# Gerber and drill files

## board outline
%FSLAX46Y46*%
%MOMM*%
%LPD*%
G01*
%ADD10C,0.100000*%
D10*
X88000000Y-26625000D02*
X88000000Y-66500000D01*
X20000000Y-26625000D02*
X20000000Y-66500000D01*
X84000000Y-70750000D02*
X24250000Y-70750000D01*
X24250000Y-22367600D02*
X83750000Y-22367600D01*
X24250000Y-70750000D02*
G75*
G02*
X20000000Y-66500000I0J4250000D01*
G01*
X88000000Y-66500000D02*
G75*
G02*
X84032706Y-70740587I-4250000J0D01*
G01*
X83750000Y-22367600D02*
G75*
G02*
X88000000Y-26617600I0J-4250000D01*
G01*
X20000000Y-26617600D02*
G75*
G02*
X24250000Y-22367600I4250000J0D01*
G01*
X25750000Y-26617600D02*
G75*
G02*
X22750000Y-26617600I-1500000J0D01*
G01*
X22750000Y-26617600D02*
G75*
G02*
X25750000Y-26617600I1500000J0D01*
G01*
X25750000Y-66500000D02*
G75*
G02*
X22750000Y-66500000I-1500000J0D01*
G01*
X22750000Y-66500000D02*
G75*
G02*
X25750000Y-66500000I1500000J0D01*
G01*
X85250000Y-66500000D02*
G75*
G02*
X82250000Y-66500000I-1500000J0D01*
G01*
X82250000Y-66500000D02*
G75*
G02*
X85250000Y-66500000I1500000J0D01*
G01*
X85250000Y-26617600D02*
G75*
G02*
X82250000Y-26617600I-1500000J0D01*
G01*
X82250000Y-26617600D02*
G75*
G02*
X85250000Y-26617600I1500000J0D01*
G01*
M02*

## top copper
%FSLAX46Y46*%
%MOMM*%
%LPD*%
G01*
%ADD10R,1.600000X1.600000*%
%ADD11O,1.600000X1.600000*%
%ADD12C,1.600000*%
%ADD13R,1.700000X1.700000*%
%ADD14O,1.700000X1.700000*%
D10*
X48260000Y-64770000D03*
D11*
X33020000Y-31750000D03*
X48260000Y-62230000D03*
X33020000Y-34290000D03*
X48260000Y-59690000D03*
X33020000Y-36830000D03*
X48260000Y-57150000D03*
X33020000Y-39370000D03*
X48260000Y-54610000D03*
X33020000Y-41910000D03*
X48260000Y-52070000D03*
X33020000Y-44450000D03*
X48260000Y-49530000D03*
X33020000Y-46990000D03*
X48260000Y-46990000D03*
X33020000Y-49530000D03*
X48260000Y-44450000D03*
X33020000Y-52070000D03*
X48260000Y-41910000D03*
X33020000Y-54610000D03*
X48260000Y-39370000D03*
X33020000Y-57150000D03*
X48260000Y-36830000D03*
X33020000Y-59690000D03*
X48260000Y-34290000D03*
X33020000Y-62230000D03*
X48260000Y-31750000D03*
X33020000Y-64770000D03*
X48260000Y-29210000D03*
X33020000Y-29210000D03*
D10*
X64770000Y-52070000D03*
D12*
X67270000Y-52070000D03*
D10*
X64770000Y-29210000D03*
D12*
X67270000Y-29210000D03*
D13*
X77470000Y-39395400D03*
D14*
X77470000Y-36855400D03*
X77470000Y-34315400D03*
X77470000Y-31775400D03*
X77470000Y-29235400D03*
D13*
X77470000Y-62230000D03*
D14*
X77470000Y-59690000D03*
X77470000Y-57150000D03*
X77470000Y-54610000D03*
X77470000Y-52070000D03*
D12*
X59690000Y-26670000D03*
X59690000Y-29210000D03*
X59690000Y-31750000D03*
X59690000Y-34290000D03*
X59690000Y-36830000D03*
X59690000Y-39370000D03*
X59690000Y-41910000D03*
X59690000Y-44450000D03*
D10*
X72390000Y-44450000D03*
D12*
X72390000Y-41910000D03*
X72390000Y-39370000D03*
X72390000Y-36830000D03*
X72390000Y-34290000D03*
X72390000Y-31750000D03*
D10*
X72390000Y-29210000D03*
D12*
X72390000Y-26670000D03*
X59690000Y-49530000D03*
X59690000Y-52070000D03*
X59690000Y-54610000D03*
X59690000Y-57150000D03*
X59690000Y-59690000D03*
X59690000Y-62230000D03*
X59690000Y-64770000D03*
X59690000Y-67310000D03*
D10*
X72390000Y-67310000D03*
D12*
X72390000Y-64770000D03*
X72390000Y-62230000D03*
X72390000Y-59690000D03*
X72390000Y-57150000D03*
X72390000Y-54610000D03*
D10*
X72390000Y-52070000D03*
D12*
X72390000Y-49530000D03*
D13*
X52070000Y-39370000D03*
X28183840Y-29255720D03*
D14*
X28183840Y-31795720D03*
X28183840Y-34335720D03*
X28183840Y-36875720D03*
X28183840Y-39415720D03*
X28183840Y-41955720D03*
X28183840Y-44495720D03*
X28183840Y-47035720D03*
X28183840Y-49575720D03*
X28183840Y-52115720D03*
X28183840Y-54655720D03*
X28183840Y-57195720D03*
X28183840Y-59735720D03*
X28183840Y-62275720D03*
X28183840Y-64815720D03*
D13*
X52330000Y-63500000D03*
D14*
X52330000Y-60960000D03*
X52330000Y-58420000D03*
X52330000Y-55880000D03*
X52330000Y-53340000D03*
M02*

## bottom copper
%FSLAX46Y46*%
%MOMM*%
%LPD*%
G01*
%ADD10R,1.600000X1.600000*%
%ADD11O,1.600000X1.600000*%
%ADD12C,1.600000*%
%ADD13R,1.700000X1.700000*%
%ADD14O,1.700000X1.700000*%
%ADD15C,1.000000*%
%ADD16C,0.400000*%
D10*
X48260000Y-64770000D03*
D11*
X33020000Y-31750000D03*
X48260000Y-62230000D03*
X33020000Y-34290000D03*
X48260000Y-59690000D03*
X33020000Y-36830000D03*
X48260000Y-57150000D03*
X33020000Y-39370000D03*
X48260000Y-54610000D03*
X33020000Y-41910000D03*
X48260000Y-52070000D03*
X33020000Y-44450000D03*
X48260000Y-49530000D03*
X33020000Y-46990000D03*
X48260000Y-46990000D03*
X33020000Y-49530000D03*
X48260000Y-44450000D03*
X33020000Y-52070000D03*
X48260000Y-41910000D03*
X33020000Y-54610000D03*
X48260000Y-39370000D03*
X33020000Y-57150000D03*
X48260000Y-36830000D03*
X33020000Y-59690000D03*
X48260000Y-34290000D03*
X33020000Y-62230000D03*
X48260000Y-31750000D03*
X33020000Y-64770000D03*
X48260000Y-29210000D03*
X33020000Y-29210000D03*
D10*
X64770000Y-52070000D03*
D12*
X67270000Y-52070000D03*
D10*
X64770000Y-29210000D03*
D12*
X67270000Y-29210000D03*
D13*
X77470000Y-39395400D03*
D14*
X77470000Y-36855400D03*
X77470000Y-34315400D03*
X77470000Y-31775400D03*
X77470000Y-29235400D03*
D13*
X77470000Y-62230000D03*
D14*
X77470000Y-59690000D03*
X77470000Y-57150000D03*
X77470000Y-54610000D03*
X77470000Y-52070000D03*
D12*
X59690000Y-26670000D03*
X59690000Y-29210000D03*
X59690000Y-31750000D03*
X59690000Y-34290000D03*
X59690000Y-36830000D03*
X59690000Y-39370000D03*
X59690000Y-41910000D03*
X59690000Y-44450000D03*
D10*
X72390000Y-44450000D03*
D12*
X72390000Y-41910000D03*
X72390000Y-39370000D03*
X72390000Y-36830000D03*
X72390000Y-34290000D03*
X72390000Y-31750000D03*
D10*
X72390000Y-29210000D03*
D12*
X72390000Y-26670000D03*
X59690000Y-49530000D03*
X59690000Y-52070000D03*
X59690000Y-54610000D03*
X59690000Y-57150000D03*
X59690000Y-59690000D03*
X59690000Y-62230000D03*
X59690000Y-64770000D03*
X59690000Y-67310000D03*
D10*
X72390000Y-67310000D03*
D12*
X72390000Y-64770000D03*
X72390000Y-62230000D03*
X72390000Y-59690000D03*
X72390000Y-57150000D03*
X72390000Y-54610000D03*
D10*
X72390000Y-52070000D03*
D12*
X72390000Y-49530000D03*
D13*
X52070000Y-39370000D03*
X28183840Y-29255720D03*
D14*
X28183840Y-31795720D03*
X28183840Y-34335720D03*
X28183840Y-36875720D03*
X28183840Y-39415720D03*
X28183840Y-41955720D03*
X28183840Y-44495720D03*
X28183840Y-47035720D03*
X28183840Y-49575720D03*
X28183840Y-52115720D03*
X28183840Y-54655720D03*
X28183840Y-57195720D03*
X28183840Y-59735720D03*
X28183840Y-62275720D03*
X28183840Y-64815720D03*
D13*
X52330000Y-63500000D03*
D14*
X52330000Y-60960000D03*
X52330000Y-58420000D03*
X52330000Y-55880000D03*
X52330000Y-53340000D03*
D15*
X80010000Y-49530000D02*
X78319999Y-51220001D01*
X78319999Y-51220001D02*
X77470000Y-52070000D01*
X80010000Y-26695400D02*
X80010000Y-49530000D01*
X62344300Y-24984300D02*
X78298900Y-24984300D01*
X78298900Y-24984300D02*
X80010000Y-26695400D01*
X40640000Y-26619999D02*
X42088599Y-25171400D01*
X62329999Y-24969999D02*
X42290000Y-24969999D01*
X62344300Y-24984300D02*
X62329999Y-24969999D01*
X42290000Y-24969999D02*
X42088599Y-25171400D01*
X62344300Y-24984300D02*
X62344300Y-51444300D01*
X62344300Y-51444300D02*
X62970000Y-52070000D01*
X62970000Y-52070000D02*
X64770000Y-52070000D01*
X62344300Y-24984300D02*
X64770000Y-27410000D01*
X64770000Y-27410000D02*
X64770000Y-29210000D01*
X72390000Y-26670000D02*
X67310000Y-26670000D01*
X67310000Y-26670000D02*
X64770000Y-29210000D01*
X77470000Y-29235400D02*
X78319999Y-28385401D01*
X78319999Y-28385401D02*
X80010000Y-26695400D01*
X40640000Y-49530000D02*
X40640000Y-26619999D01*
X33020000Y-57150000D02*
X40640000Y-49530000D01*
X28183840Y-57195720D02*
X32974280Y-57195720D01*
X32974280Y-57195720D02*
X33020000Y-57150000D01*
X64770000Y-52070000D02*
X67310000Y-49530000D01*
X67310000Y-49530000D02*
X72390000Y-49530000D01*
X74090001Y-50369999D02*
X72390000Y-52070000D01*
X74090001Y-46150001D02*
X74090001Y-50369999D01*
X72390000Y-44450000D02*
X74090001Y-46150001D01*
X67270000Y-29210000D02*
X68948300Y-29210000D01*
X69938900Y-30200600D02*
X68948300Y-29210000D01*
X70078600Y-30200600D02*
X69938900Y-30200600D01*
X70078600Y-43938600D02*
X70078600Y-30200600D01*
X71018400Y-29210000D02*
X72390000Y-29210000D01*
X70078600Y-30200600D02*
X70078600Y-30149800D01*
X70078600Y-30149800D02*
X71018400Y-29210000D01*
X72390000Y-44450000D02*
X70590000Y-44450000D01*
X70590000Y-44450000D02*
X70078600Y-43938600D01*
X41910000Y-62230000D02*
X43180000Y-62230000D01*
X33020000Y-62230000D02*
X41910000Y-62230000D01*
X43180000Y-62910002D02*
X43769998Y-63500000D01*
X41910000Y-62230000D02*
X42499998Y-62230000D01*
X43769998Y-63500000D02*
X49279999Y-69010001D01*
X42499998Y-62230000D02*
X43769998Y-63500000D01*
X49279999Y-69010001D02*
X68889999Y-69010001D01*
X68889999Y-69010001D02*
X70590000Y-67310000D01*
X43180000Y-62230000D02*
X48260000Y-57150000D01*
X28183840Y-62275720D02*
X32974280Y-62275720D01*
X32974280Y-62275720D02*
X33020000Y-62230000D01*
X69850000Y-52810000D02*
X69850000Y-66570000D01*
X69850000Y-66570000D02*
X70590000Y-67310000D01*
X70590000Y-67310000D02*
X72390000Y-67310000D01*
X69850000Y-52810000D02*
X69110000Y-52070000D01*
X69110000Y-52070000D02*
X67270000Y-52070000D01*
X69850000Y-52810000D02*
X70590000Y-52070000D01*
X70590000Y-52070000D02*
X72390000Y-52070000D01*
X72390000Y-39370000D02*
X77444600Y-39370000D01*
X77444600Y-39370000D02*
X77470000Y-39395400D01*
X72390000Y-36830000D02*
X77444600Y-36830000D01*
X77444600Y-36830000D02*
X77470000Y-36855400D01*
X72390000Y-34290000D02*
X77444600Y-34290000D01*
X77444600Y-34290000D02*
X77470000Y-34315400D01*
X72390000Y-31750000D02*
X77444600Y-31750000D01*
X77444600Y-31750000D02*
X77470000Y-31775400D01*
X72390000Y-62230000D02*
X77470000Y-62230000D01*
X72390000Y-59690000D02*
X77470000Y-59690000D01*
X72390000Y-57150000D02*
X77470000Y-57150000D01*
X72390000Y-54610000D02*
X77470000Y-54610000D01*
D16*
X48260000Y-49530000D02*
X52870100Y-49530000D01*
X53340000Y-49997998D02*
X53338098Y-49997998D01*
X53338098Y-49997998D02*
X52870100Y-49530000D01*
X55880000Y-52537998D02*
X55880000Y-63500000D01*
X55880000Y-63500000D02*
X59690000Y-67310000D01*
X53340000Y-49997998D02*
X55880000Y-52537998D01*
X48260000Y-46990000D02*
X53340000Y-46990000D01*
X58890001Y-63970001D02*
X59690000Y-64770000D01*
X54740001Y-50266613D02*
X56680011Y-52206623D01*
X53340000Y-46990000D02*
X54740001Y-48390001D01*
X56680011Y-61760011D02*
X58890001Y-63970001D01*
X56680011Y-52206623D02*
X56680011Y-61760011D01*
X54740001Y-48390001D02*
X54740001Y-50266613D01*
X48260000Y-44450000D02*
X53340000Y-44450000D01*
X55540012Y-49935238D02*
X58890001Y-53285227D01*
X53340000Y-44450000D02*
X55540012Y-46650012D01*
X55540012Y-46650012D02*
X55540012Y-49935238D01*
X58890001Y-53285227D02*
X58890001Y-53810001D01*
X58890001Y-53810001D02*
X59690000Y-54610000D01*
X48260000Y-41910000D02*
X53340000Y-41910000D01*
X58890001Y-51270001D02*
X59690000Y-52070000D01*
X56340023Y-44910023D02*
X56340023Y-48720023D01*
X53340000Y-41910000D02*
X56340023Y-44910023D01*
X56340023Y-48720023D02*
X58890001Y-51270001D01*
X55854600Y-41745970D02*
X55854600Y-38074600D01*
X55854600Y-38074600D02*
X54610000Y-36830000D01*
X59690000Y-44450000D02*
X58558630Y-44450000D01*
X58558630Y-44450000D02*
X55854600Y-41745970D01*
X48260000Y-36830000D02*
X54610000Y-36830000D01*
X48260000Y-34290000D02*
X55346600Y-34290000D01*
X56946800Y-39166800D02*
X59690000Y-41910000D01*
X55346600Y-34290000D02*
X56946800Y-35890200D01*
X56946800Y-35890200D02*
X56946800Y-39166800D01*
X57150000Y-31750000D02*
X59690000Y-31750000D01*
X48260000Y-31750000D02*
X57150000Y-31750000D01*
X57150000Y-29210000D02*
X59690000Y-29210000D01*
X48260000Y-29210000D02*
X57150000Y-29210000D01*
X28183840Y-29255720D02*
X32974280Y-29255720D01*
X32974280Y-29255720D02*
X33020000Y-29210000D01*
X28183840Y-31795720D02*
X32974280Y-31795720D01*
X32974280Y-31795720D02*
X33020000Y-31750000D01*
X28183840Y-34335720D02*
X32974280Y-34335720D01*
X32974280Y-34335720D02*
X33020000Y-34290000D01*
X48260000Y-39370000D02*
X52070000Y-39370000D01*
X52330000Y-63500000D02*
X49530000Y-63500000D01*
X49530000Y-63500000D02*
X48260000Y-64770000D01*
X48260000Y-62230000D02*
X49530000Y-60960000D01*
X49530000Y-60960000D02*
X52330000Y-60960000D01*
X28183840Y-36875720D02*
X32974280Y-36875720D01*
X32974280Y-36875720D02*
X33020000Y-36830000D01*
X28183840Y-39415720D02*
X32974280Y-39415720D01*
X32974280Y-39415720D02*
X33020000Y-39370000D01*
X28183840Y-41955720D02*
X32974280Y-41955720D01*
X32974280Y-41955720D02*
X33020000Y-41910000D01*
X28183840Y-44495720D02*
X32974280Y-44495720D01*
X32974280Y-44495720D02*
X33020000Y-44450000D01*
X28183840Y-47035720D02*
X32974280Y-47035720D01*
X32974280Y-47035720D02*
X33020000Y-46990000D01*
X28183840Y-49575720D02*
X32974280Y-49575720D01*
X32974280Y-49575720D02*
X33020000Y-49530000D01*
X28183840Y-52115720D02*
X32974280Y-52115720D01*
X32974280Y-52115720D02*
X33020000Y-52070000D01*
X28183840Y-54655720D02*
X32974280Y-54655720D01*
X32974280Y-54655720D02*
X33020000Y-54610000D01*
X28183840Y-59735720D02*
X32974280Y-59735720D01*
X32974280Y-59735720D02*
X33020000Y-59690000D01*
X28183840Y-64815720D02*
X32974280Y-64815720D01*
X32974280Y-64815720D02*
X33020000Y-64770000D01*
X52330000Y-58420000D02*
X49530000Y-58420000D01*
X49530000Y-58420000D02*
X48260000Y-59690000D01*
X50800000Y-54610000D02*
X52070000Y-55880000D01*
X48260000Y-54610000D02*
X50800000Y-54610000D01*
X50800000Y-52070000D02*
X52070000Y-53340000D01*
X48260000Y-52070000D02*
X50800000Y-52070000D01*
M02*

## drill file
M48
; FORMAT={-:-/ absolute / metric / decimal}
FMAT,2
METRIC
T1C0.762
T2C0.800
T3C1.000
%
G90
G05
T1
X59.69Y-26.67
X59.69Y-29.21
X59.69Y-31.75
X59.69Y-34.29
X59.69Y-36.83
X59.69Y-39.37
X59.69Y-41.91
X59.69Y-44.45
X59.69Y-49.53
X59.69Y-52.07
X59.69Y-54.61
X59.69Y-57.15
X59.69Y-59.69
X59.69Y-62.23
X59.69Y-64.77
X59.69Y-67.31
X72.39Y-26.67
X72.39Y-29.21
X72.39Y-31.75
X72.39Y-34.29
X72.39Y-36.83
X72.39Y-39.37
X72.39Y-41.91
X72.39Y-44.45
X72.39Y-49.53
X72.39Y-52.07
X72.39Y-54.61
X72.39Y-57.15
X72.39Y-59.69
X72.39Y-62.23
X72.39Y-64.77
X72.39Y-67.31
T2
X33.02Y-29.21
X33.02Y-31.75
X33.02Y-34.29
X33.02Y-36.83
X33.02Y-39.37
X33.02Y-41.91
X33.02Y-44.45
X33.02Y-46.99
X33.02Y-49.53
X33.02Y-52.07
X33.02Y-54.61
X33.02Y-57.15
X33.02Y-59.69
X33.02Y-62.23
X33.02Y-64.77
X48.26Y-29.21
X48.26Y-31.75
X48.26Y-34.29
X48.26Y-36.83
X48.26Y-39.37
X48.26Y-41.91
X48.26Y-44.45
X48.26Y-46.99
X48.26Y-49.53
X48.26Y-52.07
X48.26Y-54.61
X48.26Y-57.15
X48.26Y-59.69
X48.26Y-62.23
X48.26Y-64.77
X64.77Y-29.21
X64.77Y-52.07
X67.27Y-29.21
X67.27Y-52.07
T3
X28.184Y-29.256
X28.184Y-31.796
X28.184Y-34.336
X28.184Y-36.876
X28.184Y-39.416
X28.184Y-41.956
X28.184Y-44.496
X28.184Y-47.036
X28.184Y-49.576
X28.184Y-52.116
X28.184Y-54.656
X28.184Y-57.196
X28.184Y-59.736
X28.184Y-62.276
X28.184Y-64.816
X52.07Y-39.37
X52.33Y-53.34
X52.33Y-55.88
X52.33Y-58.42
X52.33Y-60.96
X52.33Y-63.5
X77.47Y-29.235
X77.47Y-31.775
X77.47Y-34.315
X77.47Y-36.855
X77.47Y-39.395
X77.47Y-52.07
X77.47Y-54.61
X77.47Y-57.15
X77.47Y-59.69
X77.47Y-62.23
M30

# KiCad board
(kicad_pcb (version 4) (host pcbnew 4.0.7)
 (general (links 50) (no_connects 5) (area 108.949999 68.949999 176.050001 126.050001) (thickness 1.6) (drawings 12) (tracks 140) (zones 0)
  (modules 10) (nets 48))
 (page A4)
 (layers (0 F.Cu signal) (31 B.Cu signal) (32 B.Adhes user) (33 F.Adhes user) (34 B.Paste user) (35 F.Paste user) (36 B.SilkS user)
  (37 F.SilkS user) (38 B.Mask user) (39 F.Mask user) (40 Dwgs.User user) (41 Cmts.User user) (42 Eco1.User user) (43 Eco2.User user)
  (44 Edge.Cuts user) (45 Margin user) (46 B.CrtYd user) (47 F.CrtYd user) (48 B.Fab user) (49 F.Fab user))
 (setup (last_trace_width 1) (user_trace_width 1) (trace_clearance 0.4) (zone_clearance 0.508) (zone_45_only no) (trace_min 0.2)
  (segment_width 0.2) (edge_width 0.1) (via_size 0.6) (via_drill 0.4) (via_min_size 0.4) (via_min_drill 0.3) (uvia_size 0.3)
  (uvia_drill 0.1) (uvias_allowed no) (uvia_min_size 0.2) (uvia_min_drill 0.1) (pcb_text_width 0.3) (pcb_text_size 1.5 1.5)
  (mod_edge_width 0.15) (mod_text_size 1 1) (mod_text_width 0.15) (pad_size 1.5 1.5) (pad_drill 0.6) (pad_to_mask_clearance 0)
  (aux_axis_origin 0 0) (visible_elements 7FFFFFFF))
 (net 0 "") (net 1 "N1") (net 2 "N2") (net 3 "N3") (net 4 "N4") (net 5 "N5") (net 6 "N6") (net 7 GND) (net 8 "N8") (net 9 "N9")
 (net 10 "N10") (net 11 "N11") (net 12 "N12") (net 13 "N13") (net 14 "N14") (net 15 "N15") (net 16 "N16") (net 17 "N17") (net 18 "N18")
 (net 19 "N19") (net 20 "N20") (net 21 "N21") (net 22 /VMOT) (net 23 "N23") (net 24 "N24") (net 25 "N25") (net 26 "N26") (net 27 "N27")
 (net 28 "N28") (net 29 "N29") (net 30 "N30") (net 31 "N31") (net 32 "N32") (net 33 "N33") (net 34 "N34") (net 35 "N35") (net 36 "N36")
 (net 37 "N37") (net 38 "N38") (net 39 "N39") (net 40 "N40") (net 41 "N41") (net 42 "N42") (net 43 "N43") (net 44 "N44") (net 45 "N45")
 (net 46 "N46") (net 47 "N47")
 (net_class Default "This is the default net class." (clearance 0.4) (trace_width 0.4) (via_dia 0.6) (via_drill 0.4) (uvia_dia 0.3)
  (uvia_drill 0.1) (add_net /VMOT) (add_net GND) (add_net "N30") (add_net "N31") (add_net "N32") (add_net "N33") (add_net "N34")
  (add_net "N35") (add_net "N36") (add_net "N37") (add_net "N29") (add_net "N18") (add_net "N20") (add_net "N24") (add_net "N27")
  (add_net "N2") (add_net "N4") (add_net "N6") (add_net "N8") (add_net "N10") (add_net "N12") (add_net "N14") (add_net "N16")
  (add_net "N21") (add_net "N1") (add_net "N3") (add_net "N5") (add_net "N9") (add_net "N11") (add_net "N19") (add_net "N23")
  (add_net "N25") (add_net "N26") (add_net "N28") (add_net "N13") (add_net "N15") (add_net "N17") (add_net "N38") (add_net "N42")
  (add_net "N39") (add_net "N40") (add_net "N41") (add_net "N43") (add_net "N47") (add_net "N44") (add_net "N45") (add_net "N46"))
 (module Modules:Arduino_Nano (layer F.Cu) (at 48.26 64.77 180)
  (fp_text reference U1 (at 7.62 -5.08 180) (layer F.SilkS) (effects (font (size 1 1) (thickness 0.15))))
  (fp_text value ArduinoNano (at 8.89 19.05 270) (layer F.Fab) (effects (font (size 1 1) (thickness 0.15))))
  (pad 1 thru_hole rect (at 0 0 180) (size 1.6 1.6) (drill 0.8) (layers *.Cu *.Mask) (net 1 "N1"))
  (pad 17 thru_hole oval (at 15.24 33.02 180) (size 1.6 1.6) (drill 0.8) (layers *.Cu *.Mask) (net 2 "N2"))
  (pad 2 thru_hole oval (at 0 2.54 180) (size 1.6 1.6) (drill 0.8) (layers *.Cu *.Mask) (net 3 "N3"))
  (pad 18 thru_hole oval (at 15.24 30.48 180) (size 1.6 1.6) (drill 0.8) (layers *.Cu *.Mask) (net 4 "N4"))
  (pad 3 thru_hole oval (at 0 5.08 180) (size 1.6 1.6) (drill 0.8) (layers *.Cu *.Mask) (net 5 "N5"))
  (pad 19 thru_hole oval (at 15.24 27.94 180) (size 1.6 1.6) (drill 0.8) (layers *.Cu *.Mask) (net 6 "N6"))
  (pad 4 thru_hole oval (at 0 7.62 180) (size 1.6 1.6) (drill 0.8) (layers *.Cu *.Mask) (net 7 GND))
  (pad 20 thru_hole oval (at 15.24 25.4 180) (size 1.6 1.6) (drill 0.8) (layers *.Cu *.Mask) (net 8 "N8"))
  (pad 5 thru_hole oval (at 0 10.16 180) (size 1.6 1.6) (drill 0.8) (layers *.Cu *.Mask) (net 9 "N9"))
  (pad 21 thru_hole oval (at 15.24 22.86 180) (size 1.6 1.6) (drill 0.8) (layers *.Cu *.Mask) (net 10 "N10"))
  (pad 6 thru_hole oval (at 0 12.7 180) (size 1.6 1.6) (drill 0.8) (layers *.Cu *.Mask) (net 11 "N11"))
  (pad 22 thru_hole oval (at 15.24 20.32 180) (size 1.6 1.6) (drill 0.8) (layers *.Cu *.Mask) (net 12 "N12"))
  (pad 7 thru_hole oval (at 0 15.24 180) (size 1.6 1.6) (drill 0.8) (layers *.Cu *.Mask) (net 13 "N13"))
  (pad 23 thru_hole oval (at 15.24 17.78 180) (size 1.6 1.6) (drill 0.8) (layers *.Cu *.Mask) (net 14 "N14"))
  (pad 8 thru_hole oval (at 0 17.78 180) (size 1.6 1.6) (drill 0.8) (layers *.Cu *.Mask) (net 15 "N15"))
  (pad 24 thru_hole oval (at 15.24 15.24 180) (size 1.6 1.6) (drill 0.8) (layers *.Cu *.Mask) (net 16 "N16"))
  (pad 9 thru_hole oval (at 0 20.32 180) (size 1.6 1.6) (drill 0.8) (layers *.Cu *.Mask) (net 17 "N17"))
  (pad 25 thru_hole oval (at 15.24 12.7 180) (size 1.6 1.6) (drill 0.8) (layers *.Cu *.Mask) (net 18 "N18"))
  (pad 10 thru_hole oval (at 0 22.86 180) (size 1.6 1.6) (drill 0.8) (layers *.Cu *.Mask) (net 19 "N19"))
  (pad 26 thru_hole oval (at 15.24 10.16 180) (size 1.6 1.6) (drill 0.8) (layers *.Cu *.Mask) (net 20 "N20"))
  (pad 11 thru_hole oval (at 0 25.4 180) (size 1.6 1.6) (drill 0.8) (layers *.Cu *.Mask) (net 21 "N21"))
  (pad 27 thru_hole oval (at 15.24 7.62 180) (size 1.6 1.6) (drill 0.8) (layers *.Cu *.Mask) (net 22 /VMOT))
  (pad 12 thru_hole oval (at 0 27.94 180) (size 1.6 1.6) (drill 0.8) (layers *.Cu *.Mask) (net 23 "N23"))
  (pad 28 thru_hole oval (at 15.24 5.08 180) (size 1.6 1.6) (drill 0.8) (layers *.Cu *.Mask) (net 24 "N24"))
  (pad 13 thru_hole oval (at 0 30.48 180) (size 1.6 1.6) (drill 0.8) (layers *.Cu *.Mask) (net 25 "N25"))
  (pad 29 thru_hole oval (at 15.24 2.54 180) (size 1.6 1.6) (drill 0.8) (layers *.Cu *.Mask) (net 7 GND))
  (pad 14 thru_hole oval (at 0 33.02 180) (size 1.6 1.6) (drill 0.8) (layers *.Cu *.Mask) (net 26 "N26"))
  (pad 30 thru_hole oval (at 15.24 0 180) (size 1.6 1.6) (drill 0.8) (layers *.Cu *.Mask) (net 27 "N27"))
  (pad 15 thru_hole oval (at 0 35.56 180) (size 1.6 1.6) (drill 0.8) (layers *.Cu *.Mask) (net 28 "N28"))
  (pad 16 thru_hole oval (at 15.24 35.56 180) (size 1.6 1.6) (drill 0.8) (layers *.Cu *.Mask) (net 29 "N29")))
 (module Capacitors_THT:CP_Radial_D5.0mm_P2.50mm (layer F.Cu) (at 64.77 52.07)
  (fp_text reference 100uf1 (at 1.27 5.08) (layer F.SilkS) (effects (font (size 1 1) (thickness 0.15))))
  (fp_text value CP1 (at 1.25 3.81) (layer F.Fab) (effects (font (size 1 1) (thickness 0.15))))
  (pad 1 thru_hole rect (at 0 0) (size 1.6 1.6) (drill 0.8) (layers *.Cu *.Mask) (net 22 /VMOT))
  (pad 2 thru_hole circle (at 2.5 0) (size 1.6 1.6) (drill 0.8) (layers *.Cu *.Mask) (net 7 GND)))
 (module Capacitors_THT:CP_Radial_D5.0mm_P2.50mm (layer F.Cu) (at 64.77 29.21)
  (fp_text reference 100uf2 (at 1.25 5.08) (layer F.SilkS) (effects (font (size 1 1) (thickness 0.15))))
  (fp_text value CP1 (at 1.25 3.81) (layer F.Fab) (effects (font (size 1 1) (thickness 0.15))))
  (pad 1 thru_hole rect (at 0 0) (size 1.6 1.6) (drill 0.8) (layers *.Cu *.Mask) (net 22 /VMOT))
  (pad 2 thru_hole circle (at 2.5 0) (size 1.6 1.6) (drill 0.8) (layers *.Cu *.Mask) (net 7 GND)))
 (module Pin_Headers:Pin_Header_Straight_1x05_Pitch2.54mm (layer F.Cu) (at 77.47 39.3954 180)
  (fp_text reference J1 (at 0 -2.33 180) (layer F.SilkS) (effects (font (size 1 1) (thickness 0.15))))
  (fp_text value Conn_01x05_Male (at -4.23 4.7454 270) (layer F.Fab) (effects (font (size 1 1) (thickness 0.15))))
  (pad 1 thru_hole rect (at 0 0 180) (size 1.7 1.7) (drill 1) (layers *.Cu *.Mask) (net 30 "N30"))
  (pad 2 thru_hole oval (at 0 2.54 180) (size 1.7 1.7) (drill 1) (layers *.Cu *.Mask) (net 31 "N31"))
  (pad 3 thru_hole oval (at 0 5.08 180) (size 1.7 1.7) (drill 1) (layers *.Cu *.Mask) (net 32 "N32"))
  (pad 4 thru_hole oval (at 0 7.62 180) (size 1.7 1.7) (drill 1) (layers *.Cu *.Mask) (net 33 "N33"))
  (pad 5 thru_hole oval (at 0 10.16 180) (size 1.7 1.7) (drill 1) (layers *.Cu *.Mask) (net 22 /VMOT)))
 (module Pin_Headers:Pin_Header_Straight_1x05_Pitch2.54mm (layer F.Cu) (at 77.47 62.23 180)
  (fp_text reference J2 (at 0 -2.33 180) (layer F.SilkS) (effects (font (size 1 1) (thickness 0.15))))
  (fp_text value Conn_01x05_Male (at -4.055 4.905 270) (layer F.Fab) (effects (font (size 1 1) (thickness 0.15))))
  (pad 1 thru_hole rect (at 0 0 180) (size 1.7 1.7) (drill 1) (layers *.Cu *.Mask) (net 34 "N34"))
  (pad 2 thru_hole oval (at 0 2.54 180) (size 1.7 1.7) (drill 1) (layers *.Cu *.Mask) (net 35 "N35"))
  (pad 3 thru_hole oval (at 0 5.08 180) (size 1.7 1.7) (drill 1) (layers *.Cu *.Mask) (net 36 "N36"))
  (pad 4 thru_hole oval (at 0 7.62 180) (size 1.7 1.7) (drill 1) (layers *.Cu *.Mask) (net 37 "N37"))
  (pad 5 thru_hole oval (at 0 10.16 180) (size 1.7 1.7) (drill 1) (layers *.Cu *.Mask) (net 22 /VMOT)))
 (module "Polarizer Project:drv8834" (layer F.Cu) (at 59.69 26.67)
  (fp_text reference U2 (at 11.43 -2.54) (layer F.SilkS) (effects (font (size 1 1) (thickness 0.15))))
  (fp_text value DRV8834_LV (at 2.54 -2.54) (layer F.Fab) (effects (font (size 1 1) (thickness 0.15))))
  (pad 1 thru_hole circle (at 0 0) (size 1.6 1.6) (drill 0.762) (layers *.Cu *.Mask) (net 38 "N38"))
  (pad 2 thru_hole circle (at 0 2.54) (size 1.6 1.6) (drill 0.762) (layers *.Cu *.Mask) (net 28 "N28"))
  (pad 3 thru_hole circle (at 0 5.08) (size 1.6 1.6) (drill 0.762) (layers *.Cu *.Mask) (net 26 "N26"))
  (pad 4 thru_hole circle (at 0 7.62) (size 1.6 1.6) (drill 0.762) (layers *.Cu *.Mask) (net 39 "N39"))
  (pad 5 thru_hole circle (at 0 10.16) (size 1.6 1.6) (drill 0.762) (layers *.Cu *.Mask) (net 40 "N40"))
  (pad 6 thru_hole circle (at 0 12.7) (size 1.6 1.6) (drill 0.762) (layers *.Cu *.Mask) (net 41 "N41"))
  (pad 7 thru_hole circle (at 0 15.24) (size 1.6 1.6) (drill 0.762) (layers *.Cu *.Mask) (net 25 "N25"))
  (pad 8 thru_hole circle (at 0 17.78) (size 1.6 1.6) (drill 0.762) (layers *.Cu *.Mask) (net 23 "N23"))
  (pad 9 thru_hole rect (at 12.7 17.78) (size 1.6 1.6) (drill 0.762) (layers *.Cu *.Mask) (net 7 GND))
  (pad 10 thru_hole circle (at 12.7 15.24) (size 1.6 1.6) (drill 0.762) (layers *.Cu *.Mask) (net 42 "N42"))
  (pad 11 thru_hole circle (at 12.7 12.7) (size 1.6 1.6) (drill 0.762) (layers *.Cu *.Mask) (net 30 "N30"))
  (pad 12 thru_hole circle (at 12.7 10.16) (size 1.6 1.6) (drill 0.762) (layers *.Cu *.Mask) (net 31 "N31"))
  (pad 13 thru_hole circle (at 12.7 7.62) (size 1.6 1.6) (drill 0.762) (layers *.Cu *.Mask) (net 32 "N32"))
  (pad 14 thru_hole circle (at 12.7 5.08) (size 1.6 1.6) (drill 0.762) (layers *.Cu *.Mask) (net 33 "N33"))
  (pad 15 thru_hole rect (at 12.7 2.54) (size 1.6 1.6) (drill 0.762) (layers *.Cu *.Mask) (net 7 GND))
  (pad 16 thru_hole circle (at 12.7 0) (size 1.6 1.6) (drill 0.762) (layers *.Cu *.Mask) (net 22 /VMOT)))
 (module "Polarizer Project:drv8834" (layer F.Cu) (at 59.69 49.53)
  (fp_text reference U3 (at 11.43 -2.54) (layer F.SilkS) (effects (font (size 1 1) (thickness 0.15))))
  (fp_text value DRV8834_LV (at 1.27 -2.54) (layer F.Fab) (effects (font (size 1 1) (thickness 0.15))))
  (pad 1 thru_hole circle (at 0 0) (size 1.6 1.6) (drill 0.762) (layers *.Cu *.Mask) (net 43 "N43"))
  (pad 2 thru_hole circle (at 0 2.54) (size 1.6 1.6) (drill 0.762) (layers *.Cu *.Mask) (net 19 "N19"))
  (pad 3 thru_hole circle (at 0 5.08) (size 1.6 1.6) (drill 0.762) (layers *.Cu *.Mask) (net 17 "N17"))
  (pad 4 thru_hole circle (at 0 7.62) (size 1.6 1.6) (drill 0.762) (layers *.Cu *.Mask) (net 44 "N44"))
  (pad 5 thru_hole circle (at 0 10.16) (size 1.6 1.6) (drill 0.762) (layers *.Cu *.Mask) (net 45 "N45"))
  (pad 6 thru_hole circle (at 0 12.7) (size 1.6 1.6) (drill 0.762) (layers *.Cu *.Mask) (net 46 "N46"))
  (pad 7 thru_hole circle (at 0 15.24) (size 1.6 1.6) (drill 0.762) (layers *.Cu *.Mask) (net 15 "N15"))
  (pad 8 thru_hole circle (at 0 17.78) (size 1.6 1.6) (drill 0.762) (layers *.Cu *.Mask) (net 13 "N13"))
  (pad 9 thru_hole rect (at 12.7 17.78) (size 1.6 1.6) (drill 0.762) (layers *.Cu *.Mask) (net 7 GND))
  (pad 10 thru_hole circle (at 12.7 15.24) (size 1.6 1.6) (drill 0.762) (layers *.Cu *.Mask) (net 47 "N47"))
  (pad 11 thru_hole circle (at 12.7 12.7) (size 1.6 1.6) (drill 0.762) (layers *.Cu *.Mask) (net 34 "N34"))
  (pad 12 thru_hole circle (at 12.7 10.16) (size 1.6 1.6) (drill 0.762) (layers *.Cu *.Mask) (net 35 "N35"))
  (pad 13 thru_hole circle (at 12.7 7.62) (size 1.6 1.6) (drill 0.762) (layers *.Cu *.Mask) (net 36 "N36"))
  (pad 14 thru_hole circle (at 12.7 5.08) (size 1.6 1.6) (drill 0.762) (layers *.Cu *.Mask) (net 37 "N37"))
  (pad 15 thru_hole rect (at 12.7 2.54) (size 1.6 1.6) (drill 0.762) (layers *.Cu *.Mask) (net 7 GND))
  (pad 16 thru_hole circle (at 12.7 0) (size 1.6 1.6) (drill 0.762) (layers *.Cu *.Mask) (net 22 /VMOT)))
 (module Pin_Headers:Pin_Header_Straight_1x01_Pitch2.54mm (layer F.Cu) (at 52.07 39.37)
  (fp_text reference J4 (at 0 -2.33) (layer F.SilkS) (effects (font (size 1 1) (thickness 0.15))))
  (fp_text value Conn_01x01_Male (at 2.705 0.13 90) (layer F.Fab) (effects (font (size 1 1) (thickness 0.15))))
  (pad 1 thru_hole rect (at 0 0) (size 1.7 1.7) (drill 1) (layers *.Cu *.Mask) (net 21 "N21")))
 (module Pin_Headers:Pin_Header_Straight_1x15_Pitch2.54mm (layer F.Cu) (at 28.18384 29.25572)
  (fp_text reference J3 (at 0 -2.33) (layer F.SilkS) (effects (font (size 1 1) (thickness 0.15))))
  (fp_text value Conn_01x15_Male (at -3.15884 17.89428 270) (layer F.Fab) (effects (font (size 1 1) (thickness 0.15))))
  (pad 1 thru_hole rect (at 0 0) (size 1.7 1.7) (drill 1) (layers *.Cu *.Mask) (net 29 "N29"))
  (pad 2 thru_hole oval (at 0 2.54) (size 1.7 1.7) (drill 1) (layers *.Cu *.Mask) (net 2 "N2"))
  (pad 3 thru_hole oval (at 0 5.08) (size 1.7 1.7) (drill 1) (layers *.Cu *.Mask) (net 4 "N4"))
  (pad 4 thru_hole oval (at 0 7.62) (size 1.7 1.7) (drill 1) (layers *.Cu *.Mask) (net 6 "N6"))
  (pad 5 thru_hole oval (at 0 10.16) (size 1.7 1.7) (drill 1) (layers *.Cu *.Mask) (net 8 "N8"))
  (pad 6 thru_hole oval (at 0 12.7) (size 1.7 1.7) (drill 1) (layers *.Cu *.Mask) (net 10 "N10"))
  (pad 7 thru_hole oval (at 0 15.24) (size 1.7 1.7) (drill 1) (layers *.Cu *.Mask) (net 12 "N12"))
  (pad 8 thru_hole oval (at 0 17.78) (size 1.7 1.7) (drill 1) (layers *.Cu *.Mask) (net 14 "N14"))
  (pad 9 thru_hole oval (at 0 20.32) (size 1.7 1.7) (drill 1) (layers *.Cu *.Mask) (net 16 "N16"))
  (pad 10 thru_hole oval (at 0 22.86) (size 1.7 1.7) (drill 1) (layers *.Cu *.Mask) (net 18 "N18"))
  (pad 11 thru_hole oval (at 0 25.4) (size 1.7 1.7) (drill 1) (layers *.Cu *.Mask) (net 20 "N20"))
  (pad 12 thru_hole oval (at 0 27.94) (size 1.7 1.7) (drill 1) (layers *.Cu *.Mask) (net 22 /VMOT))
  (pad 13 thru_hole oval (at 0 30.48) (size 1.7 1.7) (drill 1) (layers *.Cu *.Mask) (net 24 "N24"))
  (pad 14 thru_hole oval (at 0 33.02) (size 1.7 1.7) (drill 1) (layers *.Cu *.Mask) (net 7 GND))
  (pad 15 thru_hole oval (at 0 35.56) (size 1.7 1.7) (drill 1) (layers *.Cu *.Mask) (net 27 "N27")))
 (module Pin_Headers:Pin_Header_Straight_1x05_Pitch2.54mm (layer F.Cu) (at 52.33 63.5 180)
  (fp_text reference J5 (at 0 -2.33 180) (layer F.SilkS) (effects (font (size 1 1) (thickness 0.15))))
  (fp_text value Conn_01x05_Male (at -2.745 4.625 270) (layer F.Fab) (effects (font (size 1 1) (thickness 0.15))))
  (pad 1 thru_hole rect (at 0 0 180) (size 1.7 1.7) (drill 1) (layers *.Cu *.Mask) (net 1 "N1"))
  (pad 2 thru_hole oval (at 0 2.54 180) (size 1.7 1.7) (drill 1) (layers *.Cu *.Mask) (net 3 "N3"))
  (pad 3 thru_hole oval (at 0 5.08 180) (size 1.7 1.7) (drill 1) (layers *.Cu *.Mask) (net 5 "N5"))
  (pad 4 thru_hole oval (at 0 7.62 180) (size 1.7 1.7) (drill 1) (layers *.Cu *.Mask) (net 9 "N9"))
  (pad 5 thru_hole oval (at 0 10.16 180) (size 1.7 1.7) (drill 1) (layers *.Cu *.Mask) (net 11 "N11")))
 (gr_line (start 88 26.625) (end 88 66.5) (layer Edge.Cuts) (width 0.1))
 (gr_line (start 20 26.625) (end 20 66.5) (layer Edge.Cuts) (width 0.1))
 (gr_line (start 84 70.75) (end 24.25 70.75) (layer Edge.Cuts) (width 0.1))
 (gr_line (start 24.25 22.3676) (end 83.75 22.3676) (layer Edge.Cuts) (width 0.1))
 (gr_arc (start 24.25 66.5) (end 24.25 70.75) (angle 90) (layer Edge.Cuts) (width 0.1))
 (gr_arc (start 83.75 66.5) (end 88 66.5) (angle 86.18592517) (layer Edge.Cuts) (width 0.1))
 (gr_arc (start 83.75 26.6176) (end 83.75 22.3676) (angle 90) (layer Edge.Cuts) (width 0.1))
 (gr_arc (start 24.25 26.6176) (end 20 26.6176) (angle 90) (layer Edge.Cuts) (width 0.1))
 (gr_circle (center 24.25 26.6176) (end 22.75 26.6176) (layer Edge.Cuts) (width 0.1))
 (gr_circle (center 24.25 66.5) (end 22.75 66.5) (layer Edge.Cuts) (width 0.1))
 (gr_circle (center 83.75 66.5) (end 85.25 66.5) (layer Edge.Cuts) (width 0.1))
 (gr_circle (center 83.75 26.6176) (end 85.25 26.6176) (layer Edge.Cuts) (width 0.1))
 (segment (start 80.01 49.53) (end 78.319999 51.220001) (width 1) (layer B.Cu) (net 22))
 (segment (start 78.319999 51.220001) (end 77.47 52.07) (width 1) (layer B.Cu) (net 22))
 (segment (start 80.01 26.6954) (end 80.01 49.53) (width 1) (layer B.Cu) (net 22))
 (segment (start 62.3443 24.9843) (end 78.2989 24.9843) (width 1) (layer B.Cu) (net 22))
 (segment (start 78.2989 24.9843) (end 80.01 26.6954) (width 1) (layer B.Cu) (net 22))
 (segment (start 40.64 26.619999) (end 42.088599 25.1714) (width 1) (layer B.Cu) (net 22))
 (segment (start 62.329999 24.969999) (end 42.29 24.969999) (width 1) (layer B.Cu) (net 22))
 (segment (start 62.3443 24.9843) (end 62.329999 24.969999) (width 1) (layer B.Cu) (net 22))
 (segment (start 42.29 24.969999) (end 42.088599 25.1714) (width 1) (layer B.Cu) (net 22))
 (segment (start 62.3443 24.9843) (end 62.3443 51.4443) (width 1) (layer B.Cu) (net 22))
 (segment (start 62.3443 51.4443) (end 62.97 52.07) (width 1) (layer B.Cu) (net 22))
 (segment (start 62.97 52.07) (end 64.77 52.07) (width 1) (layer B.Cu) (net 22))
 (segment (start 62.3443 24.9843) (end 64.77 27.41) (width 1) (layer B.Cu) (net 22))
 (segment (start 64.77 27.41) (end 64.77 29.21) (width 1) (layer B.Cu) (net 22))
 (segment (start 72.39 26.67) (end 67.31 26.67) (width 1) (layer B.Cu) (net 22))
 (segment (start 67.31 26.67) (end 64.77 29.21) (width 1) (layer B.Cu) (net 22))
 (segment (start 77.47 29.2354) (end 78.319999 28.385401) (width 1) (layer B.Cu) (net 22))
 (segment (start 78.319999 28.385401) (end 80.01 26.6954) (width 1) (layer B.Cu) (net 22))
 (segment (start 40.64 49.53) (end 40.64 26.619999) (width 1) (layer B.Cu) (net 22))
 (segment (start 33.02 57.15) (end 40.64 49.53) (width 1) (layer B.Cu) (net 22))
 (segment (start 28.18384 57.19572) (end 32.97428 57.19572) (width 1) (layer B.Cu) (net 22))
 (segment (start 32.97428 57.19572) (end 33.02 57.15) (width 1) (layer B.Cu) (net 22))
 (segment (start 64.77 52.07) (end 67.31 49.53) (width 1) (layer B.Cu) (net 22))
 (segment (start 67.31 49.53) (end 72.39 49.53) (width 1) (layer B.Cu) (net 22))
 (segment (start 74.090001 50.369999) (end 72.39 52.07) (width 1) (layer B.Cu) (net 7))
 (segment (start 74.090001 46.150001) (end 74.090001 50.369999) (width 1) (layer B.Cu) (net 7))
 (segment (start 72.39 44.45) (end 74.090001 46.150001) (width 1) (layer B.Cu) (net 7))
 (segment (start 67.27 29.21) (end 68.9483 29.21) (width 1) (layer B.Cu) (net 7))
 (segment (start 69.9389 30.2006) (end 68.9483 29.21) (width 1) (layer B.Cu) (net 7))
 (segment (start 70.0786 30.2006) (end 69.9389 30.2006) (width 1) (layer B.Cu) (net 7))
 (segment (start 70.0786 43.9386) (end 70.0786 30.2006) (width 1) (layer B.Cu) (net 7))
 (segment (start 71.0184 29.21) (end 72.39 29.21) (width 1) (layer B.Cu) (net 7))
 (segment (start 70.0786 30.2006) (end 70.0786 30.1498) (width 1) (layer B.Cu) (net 7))
 (segment (start 70.0786 30.1498) (end 71.0184 29.21) (width 1) (layer B.Cu) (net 7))
 (segment (start 72.39 44.45) (end 70.59 44.45) (width 1) (layer B.Cu) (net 7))
 (segment (start 70.59 44.45) (end 70.0786 43.9386) (width 1) (layer B.Cu) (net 7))
 (segment (start 41.91 62.23) (end 43.18 62.23) (width 1) (layer B.Cu) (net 7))
 (segment (start 33.02 62.23) (end 41.91 62.23) (width 1) (layer B.Cu) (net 7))
 (segment (start 43.18 62.910002) (end 43.769998 63.5) (width 1) (layer B.Cu) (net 7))
 (segment (start 41.91 62.23) (end 42.499998 62.23) (width 1) (layer B.Cu) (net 7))
 (segment (start 43.769998 63.5) (end 49.279999 69.010001) (width 1) (layer B.Cu) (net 7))
 (segment (start 42.499998 62.23) (end 43.769998 63.5) (width 1) (layer B.Cu) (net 7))
 (segment (start 49.279999 69.010001) (end 68.889999 69.010001) (width 1) (layer B.Cu) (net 7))
 (segment (start 68.889999 69.010001) (end 70.59 67.31) (width 1) (layer B.Cu) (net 7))
 (segment (start 43.18 62.23) (end 48.26 57.15) (width 1) (layer B.Cu) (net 7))
 (segment (start 28.18384 62.27572) (end 32.97428 62.27572) (width 1) (layer B.Cu) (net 7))
 (segment (start 32.97428 62.27572) (end 33.02 62.23) (width 1) (layer B.Cu) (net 7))
 (segment (start 69.85 52.81) (end 69.85 66.57) (width 1) (layer B.Cu) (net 7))
 (segment (start 69.85 66.57) (end 70.59 67.31) (width 1) (layer B.Cu) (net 7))
 (segment (start 70.59 67.31) (end 72.39 67.31) (width 1) (layer B.Cu) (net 7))
 (segment (start 69.85 52.81) (end 69.11 52.07) (width 1) (layer B.Cu) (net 7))
 (segment (start 69.11 52.07) (end 67.27 52.07) (width 1) (layer B.Cu) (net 7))
 (segment (start 69.85 52.81) (end 70.59 52.07) (width 1) (layer B.Cu) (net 7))
 (segment (start 70.59 52.07) (end 72.39 52.07) (width 1) (layer B.Cu) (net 7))
 (segment (start 72.39 39.37) (end 77.4446 39.37) (width 1) (layer B.Cu) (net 30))
 (segment (start 77.4446 39.37) (end 77.47 39.3954) (width 1) (layer B.Cu) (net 30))
 (segment (start 72.39 36.83) (end 77.4446 36.83) (width 1) (layer B.Cu) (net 31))
 (segment (start 77.4446 36.83) (end 77.47 36.8554) (width 1) (layer B.Cu) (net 31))
 (segment (start 72.39 34.29) (end 77.4446 34.29) (width 1) (layer B.Cu) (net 32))
 (segment (start 77.4446 34.29) (end 77.47 34.3154) (width 1) (layer B.Cu) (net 32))
 (segment (start 72.39 31.75) (end 77.4446 31.75) (width 1) (layer B.Cu) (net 33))
 (segment (start 77.4446 31.75) (end 77.47 31.7754) (width 1) (layer B.Cu) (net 33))
 (segment (start 72.39 62.23) (end 77.47 62.23) (width 1) (layer B.Cu) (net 34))
 (segment (start 72.39 59.69) (end 77.47 59.69) (width 1) (layer B.Cu) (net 35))
 (segment (start 72.39 57.15) (end 77.47 57.15) (width 1) (layer B.Cu) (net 36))
 (segment (start 72.39 54.61) (end 77.47 54.61) (width 1) (layer B.Cu) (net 37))
 (segment (start 48.26 49.53) (end 52.8701 49.53) (width 0.4) (layer B.Cu) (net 13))
 (segment (start 53.34 49.997998) (end 53.338098 49.997998) (width 0.4) (layer B.Cu) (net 13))
 (segment (start 53.338098 49.997998) (end 52.8701 49.53) (width 0.4) (layer B.Cu) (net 13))
 (segment (start 55.88 52.537998) (end 55.88 63.5) (width 0.4) (layer B.Cu) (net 13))
 (segment (start 55.88 63.5) (end 59.69 67.31) (width 0.4) (layer B.Cu) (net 13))
 (segment (start 53.34 49.997998) (end 55.88 52.537998) (width 0.4) (layer B.Cu) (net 13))
 (segment (start 48.26 46.99) (end 53.34 46.99) (width 0.4) (layer B.Cu) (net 15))
 (segment (start 58.890001 63.970001) (end 59.69 64.77) (width 0.4) (layer B.Cu) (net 15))
 (segment (start 54.740001 50.266613) (end 56.680011 52.206623) (width 0.4) (layer B.Cu) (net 15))
 (segment (start 53.34 46.99) (end 54.740001 48.390001) (width 0.4) (layer B.Cu) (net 15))
 (segment (start 56.680011 61.760011) (end 58.890001 63.970001) (width 0.4) (layer B.Cu) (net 15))
 (segment (start 56.680011 52.206623) (end 56.680011 61.760011) (width 0.4) (layer B.Cu) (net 15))
 (segment (start 54.740001 48.390001) (end 54.740001 50.266613) (width 0.4) (layer B.Cu) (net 15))
 (segment (start 48.26 44.45) (end 53.34 44.45) (width 0.4) (layer B.Cu) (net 17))
 (segment (start 55.540012 49.935238) (end 58.890001 53.285227) (width 0.4) (layer B.Cu) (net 17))
 (segment (start 53.34 44.45) (end 55.540012 46.650012) (width 0.4) (layer B.Cu) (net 17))
 (segment (start 55.540012 46.650012) (end 55.540012 49.935238) (width 0.4) (layer B.Cu) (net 17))
 (segment (start 58.890001 53.285227) (end 58.890001 53.810001) (width 0.4) (layer B.Cu) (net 17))
 (segment (start 58.890001 53.810001) (end 59.69 54.61) (width 0.4) (layer B.Cu) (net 17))
 (segment (start 48.26 41.91) (end 53.34 41.91) (width 0.4) (layer B.Cu) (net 19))
 (segment (start 58.890001 51.270001) (end 59.69 52.07) (width 0.4) (layer B.Cu) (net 19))
 (segment (start 56.340023 44.910023) (end 56.340023 48.720023) (width 0.4) (layer B.Cu) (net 19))
 (segment (start 53.34 41.91) (end 56.340023 44.910023) (width 0.4) (layer B.Cu) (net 19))
 (segment (start 56.340023 48.720023) (end 58.890001 51.270001) (width 0.4) (layer B.Cu) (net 19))
 (segment (start 55.8546 41.74597) (end 55.8546 38.0746) (width 0.4) (layer B.Cu) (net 23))
 (segment (start 55.8546 38.0746) (end 54.61 36.83) (width 0.4) (layer B.Cu) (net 23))
 (segment (start 59.69 44.45) (end 58.55863 44.45) (width 0.4) (layer B.Cu) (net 23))
 (segment (start 58.55863 44.45) (end 55.8546 41.74597) (width 0.4) (layer B.Cu) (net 23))
 (segment (start 48.26 36.83) (end 54.61 36.83) (width 0.4) (layer B.Cu) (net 23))
 (segment (start 48.26 34.29) (end 55.3466 34.29) (width 0.4) (layer B.Cu) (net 25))
 (segment (start 56.9468 39.1668) (end 59.69 41.91) (width 0.4) (layer B.Cu) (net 25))
 (segment (start 55.3466 34.29) (end 56.9468 35.8902) (width 0.4) (layer B.Cu) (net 25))
 (segment (start 56.9468 35.8902) (end 56.9468 39.1668) (width 0.4) (layer B.Cu) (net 25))
 (segment (start 57.15 31.75) (end 59.69 31.75) (width 0.4) (layer B.Cu) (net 26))
 (segment (start 48.26 31.75) (end 57.15 31.75) (width 0.4) (layer B.Cu) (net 26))
 (segment (start 57.15 29.21) (end 59.69 29.21) (width 0.4) (layer B.Cu) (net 28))
 (segment (start 48.26 29.21) (end 57.15 29.21) (width 0.4) (layer B.Cu) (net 28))
 (segment (start 28.18384 29.25572) (end 32.97428 29.25572) (width 0.4) (layer B.Cu) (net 29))
 (segment (start 32.97428 29.25572) (end 33.02 29.21) (width 0.4) (layer B.Cu) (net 29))
 (segment (start 28.18384 31.79572) (end 32.97428 31.79572) (width 0.4) (layer B.Cu) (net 2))
 (segment (start 32.97428 31.79572) (end 33.02 31.75) (width 0.4) (layer B.Cu) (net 2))
 (segment (start 28.18384 34.33572) (end 32.97428 34.33572) (width 0.4) (layer B.Cu) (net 4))
 (segment (start 32.97428 34.33572) (end 33.02 34.29) (width 0.4) (layer B.Cu) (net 4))
 (segment (start 48.26 39.37) (end 52.07 39.37) (width 0.4) (layer B.Cu) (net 21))
 (segment (start 52.33 63.5) (end 49.53 63.5) (width 0.4) (layer B.Cu) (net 1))
 (segment (start 49.53 63.5) (end 48.26 64.77) (width 0.4) (layer B.Cu) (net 1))
 (segment (start 48.26 62.23) (end 49.53 60.96) (width 0.4) (layer B.Cu) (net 3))
 (segment (start 49.53 60.96) (end 52.33 60.96) (width 0.4) (layer B.Cu) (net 3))
 (segment (start 28.18384 36.87572) (end 32.97428 36.87572) (width 0.4) (layer B.Cu) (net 6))
 (segment (start 32.97428 36.87572) (end 33.02 36.83) (width 0.4) (layer B.Cu) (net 6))
 (segment (start 28.18384 39.41572) (end 32.97428 39.41572) (width 0.4) (layer B.Cu) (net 8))
 (segment (start 32.97428 39.41572) (end 33.02 39.37) (width 0.4) (layer B.Cu) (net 8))
 (segment (start 28.18384 41.95572) (end 32.97428 41.95572) (width 0.4) (layer B.Cu) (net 10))
 (segment (start 32.97428 41.95572) (end 33.02 41.91) (width 0.4) (layer B.Cu) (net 10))
 (segment (start 28.18384 44.49572) (end 32.97428 44.49572) (width 0.4) (layer B.Cu) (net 12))
 (segment (start 32.97428 44.49572) (end 33.02 44.45) (width 0.4) (layer B.Cu) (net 12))
 (segment (start 28.18384 47.03572) (end 32.97428 47.03572) (width 0.4) (layer B.Cu) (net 14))
 (segment (start 32.97428 47.03572) (end 33.02 46.99) (width 0.4) (layer B.Cu) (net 14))
 (segment (start 28.18384 49.57572) (end 32.97428 49.57572) (width 0.4) (layer B.Cu) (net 16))
 (segment (start 32.97428 49.57572) (end 33.02 49.53) (width 0.4) (layer B.Cu) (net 16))
 (segment (start 28.18384 52.11572) (end 32.97428 52.11572) (width 0.4) (layer B.Cu) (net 18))
 (segment (start 32.97428 52.11572) (end 33.02 52.07) (width 0.4) (layer B.Cu) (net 18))
 (segment (start 28.18384 54.65572) (end 32.97428 54.65572) (width 0.4) (layer B.Cu) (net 20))
 (segment (start 32.97428 54.65572) (end 33.02 54.61) (width 0.4) (layer B.Cu) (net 20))
 (segment (start 28.18384 59.73572) (end 32.97428 59.73572) (width 0.4) (layer B.Cu) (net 24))
 (segment (start 32.97428 59.73572) (end 33.02 59.69) (width 0.4) (layer B.Cu) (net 24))
 (segment (start 28.18384 64.81572) (end 32.97428 64.81572) (width 0.4) (layer B.Cu) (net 27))
 (segment (start 32.97428 64.81572) (end 33.02 64.77) (width 0.4) (layer B.Cu) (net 27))
 (segment (start 52.33 58.42) (end 49.53 58.42) (width 0.4) (layer B.Cu) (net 5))
 (segment (start 49.53 58.42) (end 48.26 59.69) (width 0.4) (layer B.Cu) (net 5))
 (segment (start 50.8 54.61) (end 52.07 55.88) (width 0.4) (layer B.Cu) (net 9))
 (segment (start 48.26 54.61) (end 50.8 54.61) (width 0.4) (layer B.Cu) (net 9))
 (segment (start 50.8 52.07) (end 52.07 53.34) (width 0.4) (layer B.Cu) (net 11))
 (segment (start 48.26 52.07) (end 50.8 52.07) (width 0.4) (layer B.Cu) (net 11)))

